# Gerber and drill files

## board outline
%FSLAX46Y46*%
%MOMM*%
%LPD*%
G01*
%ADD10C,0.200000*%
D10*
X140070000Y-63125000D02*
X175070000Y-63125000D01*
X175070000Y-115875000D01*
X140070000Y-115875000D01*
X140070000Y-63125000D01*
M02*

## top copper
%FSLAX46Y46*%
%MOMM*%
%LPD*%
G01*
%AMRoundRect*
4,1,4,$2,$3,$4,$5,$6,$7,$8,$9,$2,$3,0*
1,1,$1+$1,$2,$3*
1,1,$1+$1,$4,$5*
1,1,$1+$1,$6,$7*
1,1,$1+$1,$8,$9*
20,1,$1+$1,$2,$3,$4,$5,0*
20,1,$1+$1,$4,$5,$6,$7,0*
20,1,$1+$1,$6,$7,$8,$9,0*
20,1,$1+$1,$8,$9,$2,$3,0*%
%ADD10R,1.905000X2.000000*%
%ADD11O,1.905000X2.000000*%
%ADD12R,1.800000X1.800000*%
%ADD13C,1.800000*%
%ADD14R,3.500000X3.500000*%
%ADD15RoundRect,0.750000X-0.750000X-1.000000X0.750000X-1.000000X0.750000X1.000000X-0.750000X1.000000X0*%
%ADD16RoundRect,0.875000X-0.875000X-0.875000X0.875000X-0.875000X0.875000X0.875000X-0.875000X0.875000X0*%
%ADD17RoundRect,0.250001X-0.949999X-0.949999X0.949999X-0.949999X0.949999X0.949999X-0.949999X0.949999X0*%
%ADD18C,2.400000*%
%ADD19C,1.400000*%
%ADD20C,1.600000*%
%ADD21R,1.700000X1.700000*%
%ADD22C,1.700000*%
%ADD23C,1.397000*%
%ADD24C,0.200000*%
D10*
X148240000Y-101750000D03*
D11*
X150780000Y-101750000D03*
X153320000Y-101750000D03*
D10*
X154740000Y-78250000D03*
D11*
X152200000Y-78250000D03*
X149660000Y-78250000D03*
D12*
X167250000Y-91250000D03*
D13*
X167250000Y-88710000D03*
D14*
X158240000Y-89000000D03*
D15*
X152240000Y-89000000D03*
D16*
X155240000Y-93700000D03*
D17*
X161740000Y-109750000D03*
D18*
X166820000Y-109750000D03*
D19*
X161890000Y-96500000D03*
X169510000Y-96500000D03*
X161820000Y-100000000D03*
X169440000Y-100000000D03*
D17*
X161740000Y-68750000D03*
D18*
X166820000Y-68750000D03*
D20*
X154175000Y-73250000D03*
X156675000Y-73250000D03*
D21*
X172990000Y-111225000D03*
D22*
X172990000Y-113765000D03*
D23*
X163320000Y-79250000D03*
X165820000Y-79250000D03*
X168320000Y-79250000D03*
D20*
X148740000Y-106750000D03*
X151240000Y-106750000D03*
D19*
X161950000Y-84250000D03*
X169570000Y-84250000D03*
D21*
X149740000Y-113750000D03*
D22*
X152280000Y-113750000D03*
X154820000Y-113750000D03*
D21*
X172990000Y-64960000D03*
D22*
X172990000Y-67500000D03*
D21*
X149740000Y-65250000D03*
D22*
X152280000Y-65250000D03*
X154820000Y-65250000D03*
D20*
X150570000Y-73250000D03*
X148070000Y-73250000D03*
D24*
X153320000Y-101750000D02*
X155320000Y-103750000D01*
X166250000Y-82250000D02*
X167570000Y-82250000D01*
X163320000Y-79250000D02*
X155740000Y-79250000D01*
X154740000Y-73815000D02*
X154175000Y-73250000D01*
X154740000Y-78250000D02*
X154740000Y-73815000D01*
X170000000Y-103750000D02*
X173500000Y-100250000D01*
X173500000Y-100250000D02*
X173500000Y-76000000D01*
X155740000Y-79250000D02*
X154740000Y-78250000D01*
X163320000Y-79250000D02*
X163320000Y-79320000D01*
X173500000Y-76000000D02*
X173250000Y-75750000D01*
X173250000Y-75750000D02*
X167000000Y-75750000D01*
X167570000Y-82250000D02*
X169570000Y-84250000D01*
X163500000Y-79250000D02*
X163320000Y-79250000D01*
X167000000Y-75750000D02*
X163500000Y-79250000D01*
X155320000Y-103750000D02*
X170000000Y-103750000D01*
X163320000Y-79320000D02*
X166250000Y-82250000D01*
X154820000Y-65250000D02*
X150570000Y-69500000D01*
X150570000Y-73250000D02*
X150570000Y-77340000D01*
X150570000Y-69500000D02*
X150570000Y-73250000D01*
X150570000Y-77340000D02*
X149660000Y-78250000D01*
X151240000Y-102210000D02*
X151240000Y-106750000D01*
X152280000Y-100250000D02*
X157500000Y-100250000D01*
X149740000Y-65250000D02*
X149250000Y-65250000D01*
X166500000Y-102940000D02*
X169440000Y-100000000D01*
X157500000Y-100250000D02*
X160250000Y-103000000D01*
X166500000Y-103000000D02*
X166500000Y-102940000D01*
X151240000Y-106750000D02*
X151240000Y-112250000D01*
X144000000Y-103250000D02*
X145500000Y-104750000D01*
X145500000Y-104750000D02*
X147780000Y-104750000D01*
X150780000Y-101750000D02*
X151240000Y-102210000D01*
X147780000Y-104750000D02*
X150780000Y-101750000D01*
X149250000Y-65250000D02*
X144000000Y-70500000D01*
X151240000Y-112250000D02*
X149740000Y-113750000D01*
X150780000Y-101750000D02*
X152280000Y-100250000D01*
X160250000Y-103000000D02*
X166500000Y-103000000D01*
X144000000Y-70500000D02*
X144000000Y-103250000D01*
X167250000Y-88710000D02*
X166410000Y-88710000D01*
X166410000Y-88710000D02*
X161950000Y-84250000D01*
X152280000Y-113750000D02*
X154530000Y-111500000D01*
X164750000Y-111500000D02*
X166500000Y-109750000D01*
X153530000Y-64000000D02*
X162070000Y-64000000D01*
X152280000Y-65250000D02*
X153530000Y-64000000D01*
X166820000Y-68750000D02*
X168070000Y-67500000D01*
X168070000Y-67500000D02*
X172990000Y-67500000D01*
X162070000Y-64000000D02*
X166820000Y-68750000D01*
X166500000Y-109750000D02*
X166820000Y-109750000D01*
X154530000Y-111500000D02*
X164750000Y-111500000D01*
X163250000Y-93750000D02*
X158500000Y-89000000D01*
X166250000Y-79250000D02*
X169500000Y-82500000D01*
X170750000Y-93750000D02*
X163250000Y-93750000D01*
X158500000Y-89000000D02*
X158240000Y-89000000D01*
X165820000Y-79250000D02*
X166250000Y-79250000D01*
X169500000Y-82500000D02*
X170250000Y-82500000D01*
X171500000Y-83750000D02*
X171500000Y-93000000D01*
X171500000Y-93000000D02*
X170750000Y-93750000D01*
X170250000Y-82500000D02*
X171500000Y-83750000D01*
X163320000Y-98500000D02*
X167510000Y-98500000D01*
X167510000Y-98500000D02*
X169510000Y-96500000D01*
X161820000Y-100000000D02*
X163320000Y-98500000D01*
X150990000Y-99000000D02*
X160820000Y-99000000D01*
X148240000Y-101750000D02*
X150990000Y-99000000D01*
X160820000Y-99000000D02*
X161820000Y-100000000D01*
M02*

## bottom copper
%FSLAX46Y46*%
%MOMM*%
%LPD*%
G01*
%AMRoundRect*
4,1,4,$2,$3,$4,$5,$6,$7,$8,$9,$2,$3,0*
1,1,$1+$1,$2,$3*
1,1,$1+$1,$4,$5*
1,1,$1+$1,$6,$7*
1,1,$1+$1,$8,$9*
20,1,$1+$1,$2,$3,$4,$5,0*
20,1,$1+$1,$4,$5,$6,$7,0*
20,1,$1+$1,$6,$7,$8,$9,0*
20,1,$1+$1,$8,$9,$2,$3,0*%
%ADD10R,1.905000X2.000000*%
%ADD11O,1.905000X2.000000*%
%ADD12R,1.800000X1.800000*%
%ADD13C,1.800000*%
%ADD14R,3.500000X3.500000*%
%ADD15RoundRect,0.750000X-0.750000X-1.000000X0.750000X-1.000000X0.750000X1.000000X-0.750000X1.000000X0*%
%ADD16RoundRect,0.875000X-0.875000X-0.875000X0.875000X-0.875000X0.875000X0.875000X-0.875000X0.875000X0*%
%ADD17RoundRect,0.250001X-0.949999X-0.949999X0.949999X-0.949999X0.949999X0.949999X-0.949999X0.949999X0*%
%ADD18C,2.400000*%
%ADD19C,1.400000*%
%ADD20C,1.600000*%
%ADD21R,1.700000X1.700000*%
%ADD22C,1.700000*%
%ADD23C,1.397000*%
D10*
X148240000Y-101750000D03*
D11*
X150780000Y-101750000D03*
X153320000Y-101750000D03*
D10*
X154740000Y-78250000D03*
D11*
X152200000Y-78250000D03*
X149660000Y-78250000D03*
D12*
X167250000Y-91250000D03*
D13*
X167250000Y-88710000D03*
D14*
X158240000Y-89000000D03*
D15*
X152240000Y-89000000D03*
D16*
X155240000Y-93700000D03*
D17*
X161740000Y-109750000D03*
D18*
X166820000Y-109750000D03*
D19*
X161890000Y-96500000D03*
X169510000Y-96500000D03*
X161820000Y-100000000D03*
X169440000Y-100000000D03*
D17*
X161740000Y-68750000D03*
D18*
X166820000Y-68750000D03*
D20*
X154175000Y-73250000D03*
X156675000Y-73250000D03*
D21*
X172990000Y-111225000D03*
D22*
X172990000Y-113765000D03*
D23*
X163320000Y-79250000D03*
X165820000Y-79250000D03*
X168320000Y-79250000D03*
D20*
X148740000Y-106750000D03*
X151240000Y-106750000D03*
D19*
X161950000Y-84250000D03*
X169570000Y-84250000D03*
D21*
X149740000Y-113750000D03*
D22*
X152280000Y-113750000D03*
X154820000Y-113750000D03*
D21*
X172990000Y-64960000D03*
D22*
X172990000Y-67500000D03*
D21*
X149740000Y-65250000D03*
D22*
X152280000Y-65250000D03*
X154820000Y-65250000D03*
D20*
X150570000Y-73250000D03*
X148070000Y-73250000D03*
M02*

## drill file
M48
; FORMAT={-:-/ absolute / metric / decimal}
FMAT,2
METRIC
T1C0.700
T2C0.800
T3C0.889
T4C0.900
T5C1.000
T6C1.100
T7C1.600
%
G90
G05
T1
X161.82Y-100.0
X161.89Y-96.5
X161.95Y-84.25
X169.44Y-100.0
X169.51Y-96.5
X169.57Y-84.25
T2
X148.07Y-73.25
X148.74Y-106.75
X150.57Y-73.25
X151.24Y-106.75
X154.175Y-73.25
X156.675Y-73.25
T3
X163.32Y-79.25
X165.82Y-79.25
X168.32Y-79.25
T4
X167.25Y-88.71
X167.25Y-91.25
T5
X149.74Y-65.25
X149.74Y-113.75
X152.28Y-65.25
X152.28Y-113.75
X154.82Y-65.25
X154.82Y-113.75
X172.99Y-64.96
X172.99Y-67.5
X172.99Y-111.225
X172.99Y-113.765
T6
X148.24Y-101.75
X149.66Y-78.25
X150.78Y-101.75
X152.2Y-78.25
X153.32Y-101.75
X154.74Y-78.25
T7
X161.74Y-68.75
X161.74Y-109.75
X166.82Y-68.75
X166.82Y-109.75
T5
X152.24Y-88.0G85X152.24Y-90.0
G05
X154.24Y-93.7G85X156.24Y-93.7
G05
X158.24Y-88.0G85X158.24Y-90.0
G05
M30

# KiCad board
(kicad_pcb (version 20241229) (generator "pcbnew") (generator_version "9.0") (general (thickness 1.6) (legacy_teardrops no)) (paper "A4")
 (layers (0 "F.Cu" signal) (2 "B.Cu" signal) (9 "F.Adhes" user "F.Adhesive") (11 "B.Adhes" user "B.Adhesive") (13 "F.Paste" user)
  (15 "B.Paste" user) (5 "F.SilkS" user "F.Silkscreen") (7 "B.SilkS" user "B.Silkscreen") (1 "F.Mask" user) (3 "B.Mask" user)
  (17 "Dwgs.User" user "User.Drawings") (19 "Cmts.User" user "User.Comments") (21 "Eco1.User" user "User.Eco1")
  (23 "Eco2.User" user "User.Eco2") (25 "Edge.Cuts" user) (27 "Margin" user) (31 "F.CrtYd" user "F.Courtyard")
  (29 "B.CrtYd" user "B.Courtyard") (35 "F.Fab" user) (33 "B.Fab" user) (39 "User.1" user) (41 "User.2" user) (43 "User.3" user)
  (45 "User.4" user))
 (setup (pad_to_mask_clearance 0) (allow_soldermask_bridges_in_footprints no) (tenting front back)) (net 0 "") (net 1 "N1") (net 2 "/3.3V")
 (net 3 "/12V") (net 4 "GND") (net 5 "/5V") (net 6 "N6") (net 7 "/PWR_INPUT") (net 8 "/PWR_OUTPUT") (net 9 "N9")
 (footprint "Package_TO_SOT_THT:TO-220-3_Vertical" (layer "F.Cu") (at 148.24 101.75)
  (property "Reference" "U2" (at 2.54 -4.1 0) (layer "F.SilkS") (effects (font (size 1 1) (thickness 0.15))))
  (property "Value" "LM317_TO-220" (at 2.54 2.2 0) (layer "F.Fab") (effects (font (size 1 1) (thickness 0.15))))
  (pad "1" thru_hole rect (at 0 0) (size 1.905 2) (drill 1.1) (layers "*.Cu" "*.Mask") (remove_unused_layers no) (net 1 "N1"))
  (pad "2" thru_hole oval (at 2.54 0) (size 1.905 2) (drill 1.1) (layers "*.Cu" "*.Mask") (remove_unused_layers no) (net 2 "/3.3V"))
  (pad "3" thru_hole oval (at 5.08 0) (size 1.905 2) (drill 1.1) (layers "*.Cu" "*.Mask") (remove_unused_layers no) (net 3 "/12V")))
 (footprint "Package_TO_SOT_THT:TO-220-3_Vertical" (layer "F.Cu") (at 154.74 78.25 180)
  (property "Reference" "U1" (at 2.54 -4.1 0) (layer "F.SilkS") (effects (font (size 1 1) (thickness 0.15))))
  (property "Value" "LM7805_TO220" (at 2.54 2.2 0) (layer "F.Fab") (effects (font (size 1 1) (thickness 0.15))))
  (pad "1" thru_hole rect (at 0 0 180) (size 1.905 2) (drill 1.1) (layers "*.Cu" "*.Mask") (remove_unused_layers no) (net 3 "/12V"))
  (pad "2" thru_hole oval (at 2.54 0 180) (size 1.905 2) (drill 1.1) (layers "*.Cu" "*.Mask") (remove_unused_layers no) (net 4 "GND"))
  (pad "3" thru_hole oval (at 5.08 0 180) (size 1.905 2) (drill 1.1) (layers "*.Cu" "*.Mask") (remove_unused_layers no) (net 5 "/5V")))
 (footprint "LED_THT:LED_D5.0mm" (layer "F.Cu") (at 167.25 91.25 90)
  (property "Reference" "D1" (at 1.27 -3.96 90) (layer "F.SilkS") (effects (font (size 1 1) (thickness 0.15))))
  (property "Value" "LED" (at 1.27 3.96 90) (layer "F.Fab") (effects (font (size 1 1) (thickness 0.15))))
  (pad "1" thru_hole rect (at 0 0 90) (size 1.8 1.8) (drill 0.9) (layers "*.Cu" "*.Mask") (remove_unused_layers no) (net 4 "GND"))
  (pad "2" thru_hole circle (at 2.54 0 90) (size 1.8 1.8) (drill 0.9) (layers "*.Cu" "*.Mask") (remove_unused_layers no) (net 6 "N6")))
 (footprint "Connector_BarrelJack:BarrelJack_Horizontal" (layer "F.Cu") (at 158.24 89)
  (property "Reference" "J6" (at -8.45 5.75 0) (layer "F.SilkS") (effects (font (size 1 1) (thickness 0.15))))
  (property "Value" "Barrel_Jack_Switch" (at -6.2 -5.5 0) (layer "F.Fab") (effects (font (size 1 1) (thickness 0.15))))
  (pad "1" thru_hole rect (at 0 0) (size 3.5 3.5) (drill oval 1 3) (layers "*.Cu" "*.Mask") (remove_unused_layers no) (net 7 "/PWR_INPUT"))
  (pad "2" thru_hole roundrect (at -6 0) (size 3 3.5) (drill oval 1 3) (layers "*.Cu" "*.Mask") (remove_unused_layers no)
   (roundrect_rratio 0.25) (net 4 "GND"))
  (pad "3" thru_hole roundrect (at -3 4.7) (size 3.5 3.5) (drill oval 3 1) (layers "*.Cu" "*.Mask") (remove_unused_layers no)
   (roundrect_rratio 0.25) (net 4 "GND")))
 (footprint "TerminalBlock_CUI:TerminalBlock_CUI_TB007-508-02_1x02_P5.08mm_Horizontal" (layer "F.Cu") (at 161.74 109.75)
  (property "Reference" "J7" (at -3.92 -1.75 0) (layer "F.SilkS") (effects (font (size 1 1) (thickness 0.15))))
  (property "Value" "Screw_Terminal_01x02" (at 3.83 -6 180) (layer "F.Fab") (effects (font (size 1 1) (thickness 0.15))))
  (pad "1" thru_hole roundrect (at 0 0) (size 2.4 2.4) (drill 1.6) (layers "*.Cu" "*.Mask") (remove_unused_layers no)
   (roundrect_rratio 0.104167) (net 4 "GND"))
  (pad "2" thru_hole circle (at 5.08 0) (size 2.4 2.4) (drill 1.6) (layers "*.Cu" "*.Mask") (remove_unused_layers no) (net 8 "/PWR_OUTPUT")))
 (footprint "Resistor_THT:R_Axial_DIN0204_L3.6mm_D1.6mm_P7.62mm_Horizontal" (layer "F.Cu") (at 161.89 96.5)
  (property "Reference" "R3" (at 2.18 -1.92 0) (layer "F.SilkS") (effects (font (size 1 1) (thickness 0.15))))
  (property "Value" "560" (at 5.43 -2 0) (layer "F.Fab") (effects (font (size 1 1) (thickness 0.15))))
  (pad "1" thru_hole circle (at 0 0) (size 1.4 1.4) (drill 0.7) (layers "*.Cu" "*.Mask") (remove_unused_layers no) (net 4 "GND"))
  (pad "2" thru_hole circle (at 7.62 0) (size 1.4 1.4) (drill 0.7) (layers "*.Cu" "*.Mask") (remove_unused_layers no) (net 1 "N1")))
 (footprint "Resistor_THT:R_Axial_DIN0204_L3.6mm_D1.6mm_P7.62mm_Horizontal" (layer "F.Cu") (at 161.82 100)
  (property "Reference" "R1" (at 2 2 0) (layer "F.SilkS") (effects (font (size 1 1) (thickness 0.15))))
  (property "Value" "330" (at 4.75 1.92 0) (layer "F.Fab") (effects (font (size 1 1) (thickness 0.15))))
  (pad "1" thru_hole circle (at 0 0) (size 1.4 1.4) (drill 0.7) (layers "*.Cu" "*.Mask") (remove_unused_layers no) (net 1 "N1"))
  (pad "2" thru_hole circle (at 7.62 0) (size 1.4 1.4) (drill 0.7) (layers "*.Cu" "*.Mask") (remove_unused_layers no) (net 2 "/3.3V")))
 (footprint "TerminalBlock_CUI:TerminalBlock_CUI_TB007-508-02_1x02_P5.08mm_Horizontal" (layer "F.Cu") (at 161.74 68.75)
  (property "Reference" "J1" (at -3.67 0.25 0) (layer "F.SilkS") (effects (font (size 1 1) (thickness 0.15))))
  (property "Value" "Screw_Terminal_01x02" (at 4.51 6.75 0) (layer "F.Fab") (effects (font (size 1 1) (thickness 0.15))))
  (pad "1" thru_hole roundrect (at 0 0) (size 2.4 2.4) (drill 1.6) (layers "*.Cu" "*.Mask") (remove_unused_layers no)
   (roundrect_rratio 0.104167) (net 4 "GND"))
  (pad "2" thru_hole circle (at 5.08 0) (size 2.4 2.4) (drill 1.6) (layers "*.Cu" "*.Mask") (remove_unused_layers no) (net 8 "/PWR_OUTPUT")))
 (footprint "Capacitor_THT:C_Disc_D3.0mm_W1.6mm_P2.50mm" (layer "F.Cu") (at 154.175 73.25)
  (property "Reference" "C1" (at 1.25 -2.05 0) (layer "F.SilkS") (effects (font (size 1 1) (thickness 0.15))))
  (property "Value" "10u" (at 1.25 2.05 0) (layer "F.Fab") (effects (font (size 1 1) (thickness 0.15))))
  (pad "1" thru_hole circle (at 0 0) (size 1.6 1.6) (drill 0.8) (layers "*.Cu" "*.Mask") (remove_unused_layers no) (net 3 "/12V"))
  (pad "2" thru_hole circle (at 2.5 0) (size 1.6 1.6) (drill 0.8) (layers "*.Cu" "*.Mask") (remove_unused_layers no) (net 4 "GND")))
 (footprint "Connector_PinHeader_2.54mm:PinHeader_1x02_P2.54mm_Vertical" (layer "F.Cu") (at 172.99 111.225)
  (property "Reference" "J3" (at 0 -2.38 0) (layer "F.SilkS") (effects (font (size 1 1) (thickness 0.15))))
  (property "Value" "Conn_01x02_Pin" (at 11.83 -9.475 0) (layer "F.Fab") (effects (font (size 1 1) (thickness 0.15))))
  (pad "1" thru_hole rect (at 0 0) (size 1.7 1.7) (drill 1) (layers "*.Cu" "*.Mask") (remove_unused_layers no) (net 4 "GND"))
  (pad "2" thru_hole circle (at 0 2.54) (size 1.7 1.7) (drill 1) (layers "*.Cu" "*.Mask") (remove_unused_layers no) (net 8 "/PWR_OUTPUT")))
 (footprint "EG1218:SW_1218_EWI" (layer "F.Cu") (at 163.32 79.25 90)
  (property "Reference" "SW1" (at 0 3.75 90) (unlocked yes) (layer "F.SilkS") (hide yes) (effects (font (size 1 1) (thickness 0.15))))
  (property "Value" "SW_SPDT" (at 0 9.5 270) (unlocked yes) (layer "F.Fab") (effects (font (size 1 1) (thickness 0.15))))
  (pad "1" thru_hole circle (at 0 0 90) (size 1.397 1.397) (drill 0.889) (layers "*.Cu" "*.Mask") (remove_unused_layers no) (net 3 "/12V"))
  (pad "2" thru_hole circle (at 0 2.5 90) (size 1.397 1.397) (drill 0.889) (layers "*.Cu" "*.Mask") (remove_unused_layers no)
   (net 7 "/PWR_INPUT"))
  (pad "3" thru_hole circle (at 0 5 90) (size 1.397 1.397) (drill 0.889) (layers "*.Cu" "*.Mask") (remove_unused_layers no) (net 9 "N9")))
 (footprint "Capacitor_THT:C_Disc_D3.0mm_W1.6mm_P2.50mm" (layer "F.Cu") (at 148.74 106.75)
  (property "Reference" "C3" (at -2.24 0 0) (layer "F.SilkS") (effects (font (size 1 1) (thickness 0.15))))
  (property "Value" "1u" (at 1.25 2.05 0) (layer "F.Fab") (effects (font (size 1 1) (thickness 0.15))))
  (pad "1" thru_hole circle (at 0 0) (size 1.6 1.6) (drill 0.8) (layers "*.Cu" "*.Mask") (remove_unused_layers no) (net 4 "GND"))
  (pad "2" thru_hole circle (at 2.5 0) (size 1.6 1.6) (drill 0.8) (layers "*.Cu" "*.Mask") (remove_unused_layers no) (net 2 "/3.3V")))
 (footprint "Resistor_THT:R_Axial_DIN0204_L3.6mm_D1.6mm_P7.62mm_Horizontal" (layer "F.Cu") (at 161.95 84.25)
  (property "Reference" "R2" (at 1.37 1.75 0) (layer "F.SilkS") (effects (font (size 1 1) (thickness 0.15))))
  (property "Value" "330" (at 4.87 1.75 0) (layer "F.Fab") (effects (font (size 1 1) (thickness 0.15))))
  (pad "1" thru_hole circle (at 0 0) (size 1.4 1.4) (drill 0.7) (layers "*.Cu" "*.Mask") (remove_unused_layers no) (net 6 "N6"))
  (pad "2" thru_hole circle (at 7.62 0) (size 1.4 1.4) (drill 0.7) (layers "*.Cu" "*.Mask") (remove_unused_layers no) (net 3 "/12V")))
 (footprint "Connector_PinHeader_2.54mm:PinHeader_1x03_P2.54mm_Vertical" (layer "F.Cu") (at 149.74 113.75 90)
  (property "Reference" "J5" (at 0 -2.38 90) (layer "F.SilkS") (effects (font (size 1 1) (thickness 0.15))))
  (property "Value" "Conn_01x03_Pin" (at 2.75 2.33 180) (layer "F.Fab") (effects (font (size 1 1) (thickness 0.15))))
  (pad "1" thru_hole rect (at 0 0 90) (size 1.7 1.7) (drill 1) (layers "*.Cu" "*.Mask") (remove_unused_layers no) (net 2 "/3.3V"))
  (pad "2" thru_hole circle (at 0 2.54 90) (size 1.7 1.7) (drill 1) (layers "*.Cu" "*.Mask") (remove_unused_layers no) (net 8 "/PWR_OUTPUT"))
  (pad "3" thru_hole circle (at 0 5.08 90) (size 1.7 1.7) (drill 1) (layers "*.Cu" "*.Mask") (remove_unused_layers no) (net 5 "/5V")))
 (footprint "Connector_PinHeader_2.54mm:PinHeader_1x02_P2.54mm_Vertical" (layer "F.Cu") (at 172.99 64.96)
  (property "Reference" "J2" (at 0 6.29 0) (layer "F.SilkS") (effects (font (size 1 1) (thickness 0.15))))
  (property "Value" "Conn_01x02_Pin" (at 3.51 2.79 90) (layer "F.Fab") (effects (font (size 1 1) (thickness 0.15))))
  (pad "1" thru_hole rect (at 0 0) (size 1.7 1.7) (drill 1) (layers "*.Cu" "*.Mask") (remove_unused_layers no) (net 4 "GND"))
  (pad "2" thru_hole circle (at 0 2.54) (size 1.7 1.7) (drill 1) (layers "*.Cu" "*.Mask") (remove_unused_layers no) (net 8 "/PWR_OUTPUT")))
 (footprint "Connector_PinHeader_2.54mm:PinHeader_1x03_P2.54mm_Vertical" (layer "F.Cu") (at 149.74 65.25 90)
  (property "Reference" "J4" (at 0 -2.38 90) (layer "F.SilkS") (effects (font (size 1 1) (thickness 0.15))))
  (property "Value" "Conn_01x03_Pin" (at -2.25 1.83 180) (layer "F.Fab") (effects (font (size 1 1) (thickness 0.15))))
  (pad "1" thru_hole rect (at 0 0 90) (size 1.7 1.7) (drill 1) (layers "*.Cu" "*.Mask") (remove_unused_layers no) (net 2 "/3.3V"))
  (pad "2" thru_hole circle (at 0 2.54 90) (size 1.7 1.7) (drill 1) (layers "*.Cu" "*.Mask") (remove_unused_layers no) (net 8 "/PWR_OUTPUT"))
  (pad "3" thru_hole circle (at 0 5.08 90) (size 1.7 1.7) (drill 1) (layers "*.Cu" "*.Mask") (remove_unused_layers no) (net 5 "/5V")))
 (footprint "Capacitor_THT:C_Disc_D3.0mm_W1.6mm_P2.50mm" (layer "B.Cu") (at 150.57 73.25 180)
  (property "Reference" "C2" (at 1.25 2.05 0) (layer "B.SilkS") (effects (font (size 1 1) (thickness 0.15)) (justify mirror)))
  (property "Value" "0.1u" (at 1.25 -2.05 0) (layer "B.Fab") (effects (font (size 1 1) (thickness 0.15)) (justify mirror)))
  (pad "1" thru_hole circle (at 0 0 180) (size 1.6 1.6) (drill 0.8) (layers "*.Cu" "*.Mask") (remove_unused_layers no) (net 5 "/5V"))
  (pad "2" thru_hole circle (at 2.5 0 180) (size 1.6 1.6) (drill 0.8) (layers "*.Cu" "*.Mask") (remove_unused_layers no) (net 4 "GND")))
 (gr_rect (start 140.07 63.125) (end 175.07 115.875) (stroke (width 0.2) (type solid)) (fill no) (locked yes) (layer "Edge.Cuts"))
 (segment (start 153.32 101.75) (end 155.32 103.75) (width 0.2) (layer "F.Cu") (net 3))
 (segment (start 166.25 82.25) (end 167.57 82.25) (width 0.2) (layer "F.Cu") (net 3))
 (segment (start 163.32 79.25) (end 155.74 79.25) (width 0.2) (layer "F.Cu") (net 3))
 (segment (start 154.74 73.815) (end 154.175 73.25) (width 0.2) (layer "F.Cu") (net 3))
 (segment (start 154.74 78.25) (end 154.74 73.815) (width 0.2) (layer "F.Cu") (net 3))
 (segment (start 170 103.75) (end 173.5 100.25) (width 0.2) (layer "F.Cu") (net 3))
 (segment (start 173.5 100.25) (end 173.5 76) (width 0.2) (layer "F.Cu") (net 3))
 (segment (start 155.74 79.25) (end 154.74 78.25) (width 0.2) (layer "F.Cu") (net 3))
 (segment (start 163.32 79.25) (end 163.32 79.32) (width 0.2) (layer "F.Cu") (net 3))
 (segment (start 173.5 76) (end 173.25 75.75) (width 0.2) (layer "F.Cu") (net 3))
 (segment (start 173.25 75.75) (end 167 75.75) (width 0.2) (layer "F.Cu") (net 3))
 (segment (start 167.57 82.25) (end 169.57 84.25) (width 0.2) (layer "F.Cu") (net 3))
 (segment (start 163.5 79.25) (end 163.32 79.25) (width 0.2) (layer "F.Cu") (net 3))
 (segment (start 167 75.75) (end 163.5 79.25) (width 0.2) (layer "F.Cu") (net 3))
 (segment (start 155.32 103.75) (end 170 103.75) (width 0.2) (layer "F.Cu") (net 3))
 (segment (start 163.32 79.32) (end 166.25 82.25) (width 0.2) (layer "F.Cu") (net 3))
 (segment (start 154.82 65.25) (end 150.57 69.5) (width 0.2) (layer "F.Cu") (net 5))
 (segment (start 150.57 73.25) (end 150.57 77.34) (width 0.2) (layer "F.Cu") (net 5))
 (segment (start 150.57 69.5) (end 150.57 73.25) (width 0.2) (layer "F.Cu") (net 5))
 (segment (start 150.57 77.34) (end 149.66 78.25) (width 0.2) (layer "F.Cu") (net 5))
 (segment (start 151.24 102.21) (end 151.24 106.75) (width 0.2) (layer "F.Cu") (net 2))
 (segment (start 152.28 100.25) (end 157.5 100.25) (width 0.2) (layer "F.Cu") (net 2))
 (segment (start 149.74 65.25) (end 149.25 65.25) (width 0.2) (layer "F.Cu") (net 2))
 (segment (start 166.5 102.94) (end 169.44 100) (width 0.2) (layer "F.Cu") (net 2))
 (segment (start 157.5 100.25) (end 160.25 103) (width 0.2) (layer "F.Cu") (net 2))
 (segment (start 166.5 103) (end 166.5 102.94) (width 0.2) (layer "F.Cu") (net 2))
 (segment (start 151.24 106.75) (end 151.24 112.25) (width 0.2) (layer "F.Cu") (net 2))
 (segment (start 144 103.25) (end 145.5 104.75) (width 0.2) (layer "F.Cu") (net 2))
 (segment (start 145.5 104.75) (end 147.78 104.75) (width 0.2) (layer "F.Cu") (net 2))
 (segment (start 150.78 101.75) (end 151.24 102.21) (width 0.2) (layer "F.Cu") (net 2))
 (segment (start 147.78 104.75) (end 150.78 101.75) (width 0.2) (layer "F.Cu") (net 2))
 (segment (start 149.25 65.25) (end 144 70.5) (width 0.2) (layer "F.Cu") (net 2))
 (segment (start 151.24 112.25) (end 149.74 113.75) (width 0.2) (layer "F.Cu") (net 2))
 (segment (start 150.78 101.75) (end 152.28 100.25) (width 0.2) (layer "F.Cu") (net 2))
 (segment (start 160.25 103) (end 166.5 103) (width 0.2) (layer "F.Cu") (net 2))
 (segment (start 144 70.5) (end 144 103.25) (width 0.2) (layer "F.Cu") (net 2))
 (segment (start 167.25 88.71) (end 166.41 88.71) (width 0.2) (layer "F.Cu") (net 6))
 (segment (start 166.41 88.71) (end 161.95 84.25) (width 0.2) (layer "F.Cu") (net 6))
 (segment (start 152.28 113.75) (end 154.53 111.5) (width 0.2) (layer "F.Cu") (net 8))
 (segment (start 164.75 111.5) (end 166.5 109.75) (width 0.2) (layer "F.Cu") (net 8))
 (segment (start 153.53 64) (end 162.07 64) (width 0.2) (layer "F.Cu") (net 8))
 (segment (start 152.28 65.25) (end 153.53 64) (width 0.2) (layer "F.Cu") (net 8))
 (segment (start 166.82 68.75) (end 168.07 67.5) (width 0.2) (layer "F.Cu") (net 8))
 (segment (start 168.07 67.5) (end 172.99 67.5) (width 0.2) (layer "F.Cu") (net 8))
 (segment (start 162.07 64) (end 166.82 68.75) (width 0.2) (layer "F.Cu") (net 8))
 (segment (start 166.5 109.75) (end 166.82 109.75) (width 0.2) (layer "F.Cu") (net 8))
 (segment (start 154.53 111.5) (end 164.75 111.5) (width 0.2) (layer "F.Cu") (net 8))
 (segment (start 163.25 93.75) (end 158.5 89) (width 0.2) (layer "F.Cu") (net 7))
 (segment (start 166.25 79.25) (end 169.5 82.5) (width 0.2) (layer "F.Cu") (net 7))
 (segment (start 170.75 93.75) (end 163.25 93.75) (width 0.2) (layer "F.Cu") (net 7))
 (segment (start 158.5 89) (end 158.24 89) (width 0.2) (layer "F.Cu") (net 7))
 (segment (start 165.82 79.25) (end 166.25 79.25) (width 0.2) (layer "F.Cu") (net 7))
 (segment (start 169.5 82.5) (end 170.25 82.5) (width 0.2) (layer "F.Cu") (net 7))
 (segment (start 171.5 83.75) (end 171.5 93) (width 0.2) (layer "F.Cu") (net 7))
 (segment (start 171.5 93) (end 170.75 93.75) (width 0.2) (layer "F.Cu") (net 7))
 (segment (start 170.25 82.5) (end 171.5 83.75) (width 0.2) (layer "F.Cu") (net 7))
 (segment (start 163.32 98.5) (end 167.51 98.5) (width 0.2) (layer "F.Cu") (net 1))
 (segment (start 167.51 98.5) (end 169.51 96.5) (width 0.2) (layer "F.Cu") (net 1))
 (segment (start 161.82 100) (end 163.32 98.5) (width 0.2) (layer "F.Cu") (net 1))
 (segment (start 150.99 99) (end 160.82 99) (width 0.2) (layer "F.Cu") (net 1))
 (segment (start 148.24 101.75) (end 150.99 99) (width 0.2) (layer "F.Cu") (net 1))
 (segment (start 160.82 99) (end 161.82 100) (width 0.2) (layer "F.Cu") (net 1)))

